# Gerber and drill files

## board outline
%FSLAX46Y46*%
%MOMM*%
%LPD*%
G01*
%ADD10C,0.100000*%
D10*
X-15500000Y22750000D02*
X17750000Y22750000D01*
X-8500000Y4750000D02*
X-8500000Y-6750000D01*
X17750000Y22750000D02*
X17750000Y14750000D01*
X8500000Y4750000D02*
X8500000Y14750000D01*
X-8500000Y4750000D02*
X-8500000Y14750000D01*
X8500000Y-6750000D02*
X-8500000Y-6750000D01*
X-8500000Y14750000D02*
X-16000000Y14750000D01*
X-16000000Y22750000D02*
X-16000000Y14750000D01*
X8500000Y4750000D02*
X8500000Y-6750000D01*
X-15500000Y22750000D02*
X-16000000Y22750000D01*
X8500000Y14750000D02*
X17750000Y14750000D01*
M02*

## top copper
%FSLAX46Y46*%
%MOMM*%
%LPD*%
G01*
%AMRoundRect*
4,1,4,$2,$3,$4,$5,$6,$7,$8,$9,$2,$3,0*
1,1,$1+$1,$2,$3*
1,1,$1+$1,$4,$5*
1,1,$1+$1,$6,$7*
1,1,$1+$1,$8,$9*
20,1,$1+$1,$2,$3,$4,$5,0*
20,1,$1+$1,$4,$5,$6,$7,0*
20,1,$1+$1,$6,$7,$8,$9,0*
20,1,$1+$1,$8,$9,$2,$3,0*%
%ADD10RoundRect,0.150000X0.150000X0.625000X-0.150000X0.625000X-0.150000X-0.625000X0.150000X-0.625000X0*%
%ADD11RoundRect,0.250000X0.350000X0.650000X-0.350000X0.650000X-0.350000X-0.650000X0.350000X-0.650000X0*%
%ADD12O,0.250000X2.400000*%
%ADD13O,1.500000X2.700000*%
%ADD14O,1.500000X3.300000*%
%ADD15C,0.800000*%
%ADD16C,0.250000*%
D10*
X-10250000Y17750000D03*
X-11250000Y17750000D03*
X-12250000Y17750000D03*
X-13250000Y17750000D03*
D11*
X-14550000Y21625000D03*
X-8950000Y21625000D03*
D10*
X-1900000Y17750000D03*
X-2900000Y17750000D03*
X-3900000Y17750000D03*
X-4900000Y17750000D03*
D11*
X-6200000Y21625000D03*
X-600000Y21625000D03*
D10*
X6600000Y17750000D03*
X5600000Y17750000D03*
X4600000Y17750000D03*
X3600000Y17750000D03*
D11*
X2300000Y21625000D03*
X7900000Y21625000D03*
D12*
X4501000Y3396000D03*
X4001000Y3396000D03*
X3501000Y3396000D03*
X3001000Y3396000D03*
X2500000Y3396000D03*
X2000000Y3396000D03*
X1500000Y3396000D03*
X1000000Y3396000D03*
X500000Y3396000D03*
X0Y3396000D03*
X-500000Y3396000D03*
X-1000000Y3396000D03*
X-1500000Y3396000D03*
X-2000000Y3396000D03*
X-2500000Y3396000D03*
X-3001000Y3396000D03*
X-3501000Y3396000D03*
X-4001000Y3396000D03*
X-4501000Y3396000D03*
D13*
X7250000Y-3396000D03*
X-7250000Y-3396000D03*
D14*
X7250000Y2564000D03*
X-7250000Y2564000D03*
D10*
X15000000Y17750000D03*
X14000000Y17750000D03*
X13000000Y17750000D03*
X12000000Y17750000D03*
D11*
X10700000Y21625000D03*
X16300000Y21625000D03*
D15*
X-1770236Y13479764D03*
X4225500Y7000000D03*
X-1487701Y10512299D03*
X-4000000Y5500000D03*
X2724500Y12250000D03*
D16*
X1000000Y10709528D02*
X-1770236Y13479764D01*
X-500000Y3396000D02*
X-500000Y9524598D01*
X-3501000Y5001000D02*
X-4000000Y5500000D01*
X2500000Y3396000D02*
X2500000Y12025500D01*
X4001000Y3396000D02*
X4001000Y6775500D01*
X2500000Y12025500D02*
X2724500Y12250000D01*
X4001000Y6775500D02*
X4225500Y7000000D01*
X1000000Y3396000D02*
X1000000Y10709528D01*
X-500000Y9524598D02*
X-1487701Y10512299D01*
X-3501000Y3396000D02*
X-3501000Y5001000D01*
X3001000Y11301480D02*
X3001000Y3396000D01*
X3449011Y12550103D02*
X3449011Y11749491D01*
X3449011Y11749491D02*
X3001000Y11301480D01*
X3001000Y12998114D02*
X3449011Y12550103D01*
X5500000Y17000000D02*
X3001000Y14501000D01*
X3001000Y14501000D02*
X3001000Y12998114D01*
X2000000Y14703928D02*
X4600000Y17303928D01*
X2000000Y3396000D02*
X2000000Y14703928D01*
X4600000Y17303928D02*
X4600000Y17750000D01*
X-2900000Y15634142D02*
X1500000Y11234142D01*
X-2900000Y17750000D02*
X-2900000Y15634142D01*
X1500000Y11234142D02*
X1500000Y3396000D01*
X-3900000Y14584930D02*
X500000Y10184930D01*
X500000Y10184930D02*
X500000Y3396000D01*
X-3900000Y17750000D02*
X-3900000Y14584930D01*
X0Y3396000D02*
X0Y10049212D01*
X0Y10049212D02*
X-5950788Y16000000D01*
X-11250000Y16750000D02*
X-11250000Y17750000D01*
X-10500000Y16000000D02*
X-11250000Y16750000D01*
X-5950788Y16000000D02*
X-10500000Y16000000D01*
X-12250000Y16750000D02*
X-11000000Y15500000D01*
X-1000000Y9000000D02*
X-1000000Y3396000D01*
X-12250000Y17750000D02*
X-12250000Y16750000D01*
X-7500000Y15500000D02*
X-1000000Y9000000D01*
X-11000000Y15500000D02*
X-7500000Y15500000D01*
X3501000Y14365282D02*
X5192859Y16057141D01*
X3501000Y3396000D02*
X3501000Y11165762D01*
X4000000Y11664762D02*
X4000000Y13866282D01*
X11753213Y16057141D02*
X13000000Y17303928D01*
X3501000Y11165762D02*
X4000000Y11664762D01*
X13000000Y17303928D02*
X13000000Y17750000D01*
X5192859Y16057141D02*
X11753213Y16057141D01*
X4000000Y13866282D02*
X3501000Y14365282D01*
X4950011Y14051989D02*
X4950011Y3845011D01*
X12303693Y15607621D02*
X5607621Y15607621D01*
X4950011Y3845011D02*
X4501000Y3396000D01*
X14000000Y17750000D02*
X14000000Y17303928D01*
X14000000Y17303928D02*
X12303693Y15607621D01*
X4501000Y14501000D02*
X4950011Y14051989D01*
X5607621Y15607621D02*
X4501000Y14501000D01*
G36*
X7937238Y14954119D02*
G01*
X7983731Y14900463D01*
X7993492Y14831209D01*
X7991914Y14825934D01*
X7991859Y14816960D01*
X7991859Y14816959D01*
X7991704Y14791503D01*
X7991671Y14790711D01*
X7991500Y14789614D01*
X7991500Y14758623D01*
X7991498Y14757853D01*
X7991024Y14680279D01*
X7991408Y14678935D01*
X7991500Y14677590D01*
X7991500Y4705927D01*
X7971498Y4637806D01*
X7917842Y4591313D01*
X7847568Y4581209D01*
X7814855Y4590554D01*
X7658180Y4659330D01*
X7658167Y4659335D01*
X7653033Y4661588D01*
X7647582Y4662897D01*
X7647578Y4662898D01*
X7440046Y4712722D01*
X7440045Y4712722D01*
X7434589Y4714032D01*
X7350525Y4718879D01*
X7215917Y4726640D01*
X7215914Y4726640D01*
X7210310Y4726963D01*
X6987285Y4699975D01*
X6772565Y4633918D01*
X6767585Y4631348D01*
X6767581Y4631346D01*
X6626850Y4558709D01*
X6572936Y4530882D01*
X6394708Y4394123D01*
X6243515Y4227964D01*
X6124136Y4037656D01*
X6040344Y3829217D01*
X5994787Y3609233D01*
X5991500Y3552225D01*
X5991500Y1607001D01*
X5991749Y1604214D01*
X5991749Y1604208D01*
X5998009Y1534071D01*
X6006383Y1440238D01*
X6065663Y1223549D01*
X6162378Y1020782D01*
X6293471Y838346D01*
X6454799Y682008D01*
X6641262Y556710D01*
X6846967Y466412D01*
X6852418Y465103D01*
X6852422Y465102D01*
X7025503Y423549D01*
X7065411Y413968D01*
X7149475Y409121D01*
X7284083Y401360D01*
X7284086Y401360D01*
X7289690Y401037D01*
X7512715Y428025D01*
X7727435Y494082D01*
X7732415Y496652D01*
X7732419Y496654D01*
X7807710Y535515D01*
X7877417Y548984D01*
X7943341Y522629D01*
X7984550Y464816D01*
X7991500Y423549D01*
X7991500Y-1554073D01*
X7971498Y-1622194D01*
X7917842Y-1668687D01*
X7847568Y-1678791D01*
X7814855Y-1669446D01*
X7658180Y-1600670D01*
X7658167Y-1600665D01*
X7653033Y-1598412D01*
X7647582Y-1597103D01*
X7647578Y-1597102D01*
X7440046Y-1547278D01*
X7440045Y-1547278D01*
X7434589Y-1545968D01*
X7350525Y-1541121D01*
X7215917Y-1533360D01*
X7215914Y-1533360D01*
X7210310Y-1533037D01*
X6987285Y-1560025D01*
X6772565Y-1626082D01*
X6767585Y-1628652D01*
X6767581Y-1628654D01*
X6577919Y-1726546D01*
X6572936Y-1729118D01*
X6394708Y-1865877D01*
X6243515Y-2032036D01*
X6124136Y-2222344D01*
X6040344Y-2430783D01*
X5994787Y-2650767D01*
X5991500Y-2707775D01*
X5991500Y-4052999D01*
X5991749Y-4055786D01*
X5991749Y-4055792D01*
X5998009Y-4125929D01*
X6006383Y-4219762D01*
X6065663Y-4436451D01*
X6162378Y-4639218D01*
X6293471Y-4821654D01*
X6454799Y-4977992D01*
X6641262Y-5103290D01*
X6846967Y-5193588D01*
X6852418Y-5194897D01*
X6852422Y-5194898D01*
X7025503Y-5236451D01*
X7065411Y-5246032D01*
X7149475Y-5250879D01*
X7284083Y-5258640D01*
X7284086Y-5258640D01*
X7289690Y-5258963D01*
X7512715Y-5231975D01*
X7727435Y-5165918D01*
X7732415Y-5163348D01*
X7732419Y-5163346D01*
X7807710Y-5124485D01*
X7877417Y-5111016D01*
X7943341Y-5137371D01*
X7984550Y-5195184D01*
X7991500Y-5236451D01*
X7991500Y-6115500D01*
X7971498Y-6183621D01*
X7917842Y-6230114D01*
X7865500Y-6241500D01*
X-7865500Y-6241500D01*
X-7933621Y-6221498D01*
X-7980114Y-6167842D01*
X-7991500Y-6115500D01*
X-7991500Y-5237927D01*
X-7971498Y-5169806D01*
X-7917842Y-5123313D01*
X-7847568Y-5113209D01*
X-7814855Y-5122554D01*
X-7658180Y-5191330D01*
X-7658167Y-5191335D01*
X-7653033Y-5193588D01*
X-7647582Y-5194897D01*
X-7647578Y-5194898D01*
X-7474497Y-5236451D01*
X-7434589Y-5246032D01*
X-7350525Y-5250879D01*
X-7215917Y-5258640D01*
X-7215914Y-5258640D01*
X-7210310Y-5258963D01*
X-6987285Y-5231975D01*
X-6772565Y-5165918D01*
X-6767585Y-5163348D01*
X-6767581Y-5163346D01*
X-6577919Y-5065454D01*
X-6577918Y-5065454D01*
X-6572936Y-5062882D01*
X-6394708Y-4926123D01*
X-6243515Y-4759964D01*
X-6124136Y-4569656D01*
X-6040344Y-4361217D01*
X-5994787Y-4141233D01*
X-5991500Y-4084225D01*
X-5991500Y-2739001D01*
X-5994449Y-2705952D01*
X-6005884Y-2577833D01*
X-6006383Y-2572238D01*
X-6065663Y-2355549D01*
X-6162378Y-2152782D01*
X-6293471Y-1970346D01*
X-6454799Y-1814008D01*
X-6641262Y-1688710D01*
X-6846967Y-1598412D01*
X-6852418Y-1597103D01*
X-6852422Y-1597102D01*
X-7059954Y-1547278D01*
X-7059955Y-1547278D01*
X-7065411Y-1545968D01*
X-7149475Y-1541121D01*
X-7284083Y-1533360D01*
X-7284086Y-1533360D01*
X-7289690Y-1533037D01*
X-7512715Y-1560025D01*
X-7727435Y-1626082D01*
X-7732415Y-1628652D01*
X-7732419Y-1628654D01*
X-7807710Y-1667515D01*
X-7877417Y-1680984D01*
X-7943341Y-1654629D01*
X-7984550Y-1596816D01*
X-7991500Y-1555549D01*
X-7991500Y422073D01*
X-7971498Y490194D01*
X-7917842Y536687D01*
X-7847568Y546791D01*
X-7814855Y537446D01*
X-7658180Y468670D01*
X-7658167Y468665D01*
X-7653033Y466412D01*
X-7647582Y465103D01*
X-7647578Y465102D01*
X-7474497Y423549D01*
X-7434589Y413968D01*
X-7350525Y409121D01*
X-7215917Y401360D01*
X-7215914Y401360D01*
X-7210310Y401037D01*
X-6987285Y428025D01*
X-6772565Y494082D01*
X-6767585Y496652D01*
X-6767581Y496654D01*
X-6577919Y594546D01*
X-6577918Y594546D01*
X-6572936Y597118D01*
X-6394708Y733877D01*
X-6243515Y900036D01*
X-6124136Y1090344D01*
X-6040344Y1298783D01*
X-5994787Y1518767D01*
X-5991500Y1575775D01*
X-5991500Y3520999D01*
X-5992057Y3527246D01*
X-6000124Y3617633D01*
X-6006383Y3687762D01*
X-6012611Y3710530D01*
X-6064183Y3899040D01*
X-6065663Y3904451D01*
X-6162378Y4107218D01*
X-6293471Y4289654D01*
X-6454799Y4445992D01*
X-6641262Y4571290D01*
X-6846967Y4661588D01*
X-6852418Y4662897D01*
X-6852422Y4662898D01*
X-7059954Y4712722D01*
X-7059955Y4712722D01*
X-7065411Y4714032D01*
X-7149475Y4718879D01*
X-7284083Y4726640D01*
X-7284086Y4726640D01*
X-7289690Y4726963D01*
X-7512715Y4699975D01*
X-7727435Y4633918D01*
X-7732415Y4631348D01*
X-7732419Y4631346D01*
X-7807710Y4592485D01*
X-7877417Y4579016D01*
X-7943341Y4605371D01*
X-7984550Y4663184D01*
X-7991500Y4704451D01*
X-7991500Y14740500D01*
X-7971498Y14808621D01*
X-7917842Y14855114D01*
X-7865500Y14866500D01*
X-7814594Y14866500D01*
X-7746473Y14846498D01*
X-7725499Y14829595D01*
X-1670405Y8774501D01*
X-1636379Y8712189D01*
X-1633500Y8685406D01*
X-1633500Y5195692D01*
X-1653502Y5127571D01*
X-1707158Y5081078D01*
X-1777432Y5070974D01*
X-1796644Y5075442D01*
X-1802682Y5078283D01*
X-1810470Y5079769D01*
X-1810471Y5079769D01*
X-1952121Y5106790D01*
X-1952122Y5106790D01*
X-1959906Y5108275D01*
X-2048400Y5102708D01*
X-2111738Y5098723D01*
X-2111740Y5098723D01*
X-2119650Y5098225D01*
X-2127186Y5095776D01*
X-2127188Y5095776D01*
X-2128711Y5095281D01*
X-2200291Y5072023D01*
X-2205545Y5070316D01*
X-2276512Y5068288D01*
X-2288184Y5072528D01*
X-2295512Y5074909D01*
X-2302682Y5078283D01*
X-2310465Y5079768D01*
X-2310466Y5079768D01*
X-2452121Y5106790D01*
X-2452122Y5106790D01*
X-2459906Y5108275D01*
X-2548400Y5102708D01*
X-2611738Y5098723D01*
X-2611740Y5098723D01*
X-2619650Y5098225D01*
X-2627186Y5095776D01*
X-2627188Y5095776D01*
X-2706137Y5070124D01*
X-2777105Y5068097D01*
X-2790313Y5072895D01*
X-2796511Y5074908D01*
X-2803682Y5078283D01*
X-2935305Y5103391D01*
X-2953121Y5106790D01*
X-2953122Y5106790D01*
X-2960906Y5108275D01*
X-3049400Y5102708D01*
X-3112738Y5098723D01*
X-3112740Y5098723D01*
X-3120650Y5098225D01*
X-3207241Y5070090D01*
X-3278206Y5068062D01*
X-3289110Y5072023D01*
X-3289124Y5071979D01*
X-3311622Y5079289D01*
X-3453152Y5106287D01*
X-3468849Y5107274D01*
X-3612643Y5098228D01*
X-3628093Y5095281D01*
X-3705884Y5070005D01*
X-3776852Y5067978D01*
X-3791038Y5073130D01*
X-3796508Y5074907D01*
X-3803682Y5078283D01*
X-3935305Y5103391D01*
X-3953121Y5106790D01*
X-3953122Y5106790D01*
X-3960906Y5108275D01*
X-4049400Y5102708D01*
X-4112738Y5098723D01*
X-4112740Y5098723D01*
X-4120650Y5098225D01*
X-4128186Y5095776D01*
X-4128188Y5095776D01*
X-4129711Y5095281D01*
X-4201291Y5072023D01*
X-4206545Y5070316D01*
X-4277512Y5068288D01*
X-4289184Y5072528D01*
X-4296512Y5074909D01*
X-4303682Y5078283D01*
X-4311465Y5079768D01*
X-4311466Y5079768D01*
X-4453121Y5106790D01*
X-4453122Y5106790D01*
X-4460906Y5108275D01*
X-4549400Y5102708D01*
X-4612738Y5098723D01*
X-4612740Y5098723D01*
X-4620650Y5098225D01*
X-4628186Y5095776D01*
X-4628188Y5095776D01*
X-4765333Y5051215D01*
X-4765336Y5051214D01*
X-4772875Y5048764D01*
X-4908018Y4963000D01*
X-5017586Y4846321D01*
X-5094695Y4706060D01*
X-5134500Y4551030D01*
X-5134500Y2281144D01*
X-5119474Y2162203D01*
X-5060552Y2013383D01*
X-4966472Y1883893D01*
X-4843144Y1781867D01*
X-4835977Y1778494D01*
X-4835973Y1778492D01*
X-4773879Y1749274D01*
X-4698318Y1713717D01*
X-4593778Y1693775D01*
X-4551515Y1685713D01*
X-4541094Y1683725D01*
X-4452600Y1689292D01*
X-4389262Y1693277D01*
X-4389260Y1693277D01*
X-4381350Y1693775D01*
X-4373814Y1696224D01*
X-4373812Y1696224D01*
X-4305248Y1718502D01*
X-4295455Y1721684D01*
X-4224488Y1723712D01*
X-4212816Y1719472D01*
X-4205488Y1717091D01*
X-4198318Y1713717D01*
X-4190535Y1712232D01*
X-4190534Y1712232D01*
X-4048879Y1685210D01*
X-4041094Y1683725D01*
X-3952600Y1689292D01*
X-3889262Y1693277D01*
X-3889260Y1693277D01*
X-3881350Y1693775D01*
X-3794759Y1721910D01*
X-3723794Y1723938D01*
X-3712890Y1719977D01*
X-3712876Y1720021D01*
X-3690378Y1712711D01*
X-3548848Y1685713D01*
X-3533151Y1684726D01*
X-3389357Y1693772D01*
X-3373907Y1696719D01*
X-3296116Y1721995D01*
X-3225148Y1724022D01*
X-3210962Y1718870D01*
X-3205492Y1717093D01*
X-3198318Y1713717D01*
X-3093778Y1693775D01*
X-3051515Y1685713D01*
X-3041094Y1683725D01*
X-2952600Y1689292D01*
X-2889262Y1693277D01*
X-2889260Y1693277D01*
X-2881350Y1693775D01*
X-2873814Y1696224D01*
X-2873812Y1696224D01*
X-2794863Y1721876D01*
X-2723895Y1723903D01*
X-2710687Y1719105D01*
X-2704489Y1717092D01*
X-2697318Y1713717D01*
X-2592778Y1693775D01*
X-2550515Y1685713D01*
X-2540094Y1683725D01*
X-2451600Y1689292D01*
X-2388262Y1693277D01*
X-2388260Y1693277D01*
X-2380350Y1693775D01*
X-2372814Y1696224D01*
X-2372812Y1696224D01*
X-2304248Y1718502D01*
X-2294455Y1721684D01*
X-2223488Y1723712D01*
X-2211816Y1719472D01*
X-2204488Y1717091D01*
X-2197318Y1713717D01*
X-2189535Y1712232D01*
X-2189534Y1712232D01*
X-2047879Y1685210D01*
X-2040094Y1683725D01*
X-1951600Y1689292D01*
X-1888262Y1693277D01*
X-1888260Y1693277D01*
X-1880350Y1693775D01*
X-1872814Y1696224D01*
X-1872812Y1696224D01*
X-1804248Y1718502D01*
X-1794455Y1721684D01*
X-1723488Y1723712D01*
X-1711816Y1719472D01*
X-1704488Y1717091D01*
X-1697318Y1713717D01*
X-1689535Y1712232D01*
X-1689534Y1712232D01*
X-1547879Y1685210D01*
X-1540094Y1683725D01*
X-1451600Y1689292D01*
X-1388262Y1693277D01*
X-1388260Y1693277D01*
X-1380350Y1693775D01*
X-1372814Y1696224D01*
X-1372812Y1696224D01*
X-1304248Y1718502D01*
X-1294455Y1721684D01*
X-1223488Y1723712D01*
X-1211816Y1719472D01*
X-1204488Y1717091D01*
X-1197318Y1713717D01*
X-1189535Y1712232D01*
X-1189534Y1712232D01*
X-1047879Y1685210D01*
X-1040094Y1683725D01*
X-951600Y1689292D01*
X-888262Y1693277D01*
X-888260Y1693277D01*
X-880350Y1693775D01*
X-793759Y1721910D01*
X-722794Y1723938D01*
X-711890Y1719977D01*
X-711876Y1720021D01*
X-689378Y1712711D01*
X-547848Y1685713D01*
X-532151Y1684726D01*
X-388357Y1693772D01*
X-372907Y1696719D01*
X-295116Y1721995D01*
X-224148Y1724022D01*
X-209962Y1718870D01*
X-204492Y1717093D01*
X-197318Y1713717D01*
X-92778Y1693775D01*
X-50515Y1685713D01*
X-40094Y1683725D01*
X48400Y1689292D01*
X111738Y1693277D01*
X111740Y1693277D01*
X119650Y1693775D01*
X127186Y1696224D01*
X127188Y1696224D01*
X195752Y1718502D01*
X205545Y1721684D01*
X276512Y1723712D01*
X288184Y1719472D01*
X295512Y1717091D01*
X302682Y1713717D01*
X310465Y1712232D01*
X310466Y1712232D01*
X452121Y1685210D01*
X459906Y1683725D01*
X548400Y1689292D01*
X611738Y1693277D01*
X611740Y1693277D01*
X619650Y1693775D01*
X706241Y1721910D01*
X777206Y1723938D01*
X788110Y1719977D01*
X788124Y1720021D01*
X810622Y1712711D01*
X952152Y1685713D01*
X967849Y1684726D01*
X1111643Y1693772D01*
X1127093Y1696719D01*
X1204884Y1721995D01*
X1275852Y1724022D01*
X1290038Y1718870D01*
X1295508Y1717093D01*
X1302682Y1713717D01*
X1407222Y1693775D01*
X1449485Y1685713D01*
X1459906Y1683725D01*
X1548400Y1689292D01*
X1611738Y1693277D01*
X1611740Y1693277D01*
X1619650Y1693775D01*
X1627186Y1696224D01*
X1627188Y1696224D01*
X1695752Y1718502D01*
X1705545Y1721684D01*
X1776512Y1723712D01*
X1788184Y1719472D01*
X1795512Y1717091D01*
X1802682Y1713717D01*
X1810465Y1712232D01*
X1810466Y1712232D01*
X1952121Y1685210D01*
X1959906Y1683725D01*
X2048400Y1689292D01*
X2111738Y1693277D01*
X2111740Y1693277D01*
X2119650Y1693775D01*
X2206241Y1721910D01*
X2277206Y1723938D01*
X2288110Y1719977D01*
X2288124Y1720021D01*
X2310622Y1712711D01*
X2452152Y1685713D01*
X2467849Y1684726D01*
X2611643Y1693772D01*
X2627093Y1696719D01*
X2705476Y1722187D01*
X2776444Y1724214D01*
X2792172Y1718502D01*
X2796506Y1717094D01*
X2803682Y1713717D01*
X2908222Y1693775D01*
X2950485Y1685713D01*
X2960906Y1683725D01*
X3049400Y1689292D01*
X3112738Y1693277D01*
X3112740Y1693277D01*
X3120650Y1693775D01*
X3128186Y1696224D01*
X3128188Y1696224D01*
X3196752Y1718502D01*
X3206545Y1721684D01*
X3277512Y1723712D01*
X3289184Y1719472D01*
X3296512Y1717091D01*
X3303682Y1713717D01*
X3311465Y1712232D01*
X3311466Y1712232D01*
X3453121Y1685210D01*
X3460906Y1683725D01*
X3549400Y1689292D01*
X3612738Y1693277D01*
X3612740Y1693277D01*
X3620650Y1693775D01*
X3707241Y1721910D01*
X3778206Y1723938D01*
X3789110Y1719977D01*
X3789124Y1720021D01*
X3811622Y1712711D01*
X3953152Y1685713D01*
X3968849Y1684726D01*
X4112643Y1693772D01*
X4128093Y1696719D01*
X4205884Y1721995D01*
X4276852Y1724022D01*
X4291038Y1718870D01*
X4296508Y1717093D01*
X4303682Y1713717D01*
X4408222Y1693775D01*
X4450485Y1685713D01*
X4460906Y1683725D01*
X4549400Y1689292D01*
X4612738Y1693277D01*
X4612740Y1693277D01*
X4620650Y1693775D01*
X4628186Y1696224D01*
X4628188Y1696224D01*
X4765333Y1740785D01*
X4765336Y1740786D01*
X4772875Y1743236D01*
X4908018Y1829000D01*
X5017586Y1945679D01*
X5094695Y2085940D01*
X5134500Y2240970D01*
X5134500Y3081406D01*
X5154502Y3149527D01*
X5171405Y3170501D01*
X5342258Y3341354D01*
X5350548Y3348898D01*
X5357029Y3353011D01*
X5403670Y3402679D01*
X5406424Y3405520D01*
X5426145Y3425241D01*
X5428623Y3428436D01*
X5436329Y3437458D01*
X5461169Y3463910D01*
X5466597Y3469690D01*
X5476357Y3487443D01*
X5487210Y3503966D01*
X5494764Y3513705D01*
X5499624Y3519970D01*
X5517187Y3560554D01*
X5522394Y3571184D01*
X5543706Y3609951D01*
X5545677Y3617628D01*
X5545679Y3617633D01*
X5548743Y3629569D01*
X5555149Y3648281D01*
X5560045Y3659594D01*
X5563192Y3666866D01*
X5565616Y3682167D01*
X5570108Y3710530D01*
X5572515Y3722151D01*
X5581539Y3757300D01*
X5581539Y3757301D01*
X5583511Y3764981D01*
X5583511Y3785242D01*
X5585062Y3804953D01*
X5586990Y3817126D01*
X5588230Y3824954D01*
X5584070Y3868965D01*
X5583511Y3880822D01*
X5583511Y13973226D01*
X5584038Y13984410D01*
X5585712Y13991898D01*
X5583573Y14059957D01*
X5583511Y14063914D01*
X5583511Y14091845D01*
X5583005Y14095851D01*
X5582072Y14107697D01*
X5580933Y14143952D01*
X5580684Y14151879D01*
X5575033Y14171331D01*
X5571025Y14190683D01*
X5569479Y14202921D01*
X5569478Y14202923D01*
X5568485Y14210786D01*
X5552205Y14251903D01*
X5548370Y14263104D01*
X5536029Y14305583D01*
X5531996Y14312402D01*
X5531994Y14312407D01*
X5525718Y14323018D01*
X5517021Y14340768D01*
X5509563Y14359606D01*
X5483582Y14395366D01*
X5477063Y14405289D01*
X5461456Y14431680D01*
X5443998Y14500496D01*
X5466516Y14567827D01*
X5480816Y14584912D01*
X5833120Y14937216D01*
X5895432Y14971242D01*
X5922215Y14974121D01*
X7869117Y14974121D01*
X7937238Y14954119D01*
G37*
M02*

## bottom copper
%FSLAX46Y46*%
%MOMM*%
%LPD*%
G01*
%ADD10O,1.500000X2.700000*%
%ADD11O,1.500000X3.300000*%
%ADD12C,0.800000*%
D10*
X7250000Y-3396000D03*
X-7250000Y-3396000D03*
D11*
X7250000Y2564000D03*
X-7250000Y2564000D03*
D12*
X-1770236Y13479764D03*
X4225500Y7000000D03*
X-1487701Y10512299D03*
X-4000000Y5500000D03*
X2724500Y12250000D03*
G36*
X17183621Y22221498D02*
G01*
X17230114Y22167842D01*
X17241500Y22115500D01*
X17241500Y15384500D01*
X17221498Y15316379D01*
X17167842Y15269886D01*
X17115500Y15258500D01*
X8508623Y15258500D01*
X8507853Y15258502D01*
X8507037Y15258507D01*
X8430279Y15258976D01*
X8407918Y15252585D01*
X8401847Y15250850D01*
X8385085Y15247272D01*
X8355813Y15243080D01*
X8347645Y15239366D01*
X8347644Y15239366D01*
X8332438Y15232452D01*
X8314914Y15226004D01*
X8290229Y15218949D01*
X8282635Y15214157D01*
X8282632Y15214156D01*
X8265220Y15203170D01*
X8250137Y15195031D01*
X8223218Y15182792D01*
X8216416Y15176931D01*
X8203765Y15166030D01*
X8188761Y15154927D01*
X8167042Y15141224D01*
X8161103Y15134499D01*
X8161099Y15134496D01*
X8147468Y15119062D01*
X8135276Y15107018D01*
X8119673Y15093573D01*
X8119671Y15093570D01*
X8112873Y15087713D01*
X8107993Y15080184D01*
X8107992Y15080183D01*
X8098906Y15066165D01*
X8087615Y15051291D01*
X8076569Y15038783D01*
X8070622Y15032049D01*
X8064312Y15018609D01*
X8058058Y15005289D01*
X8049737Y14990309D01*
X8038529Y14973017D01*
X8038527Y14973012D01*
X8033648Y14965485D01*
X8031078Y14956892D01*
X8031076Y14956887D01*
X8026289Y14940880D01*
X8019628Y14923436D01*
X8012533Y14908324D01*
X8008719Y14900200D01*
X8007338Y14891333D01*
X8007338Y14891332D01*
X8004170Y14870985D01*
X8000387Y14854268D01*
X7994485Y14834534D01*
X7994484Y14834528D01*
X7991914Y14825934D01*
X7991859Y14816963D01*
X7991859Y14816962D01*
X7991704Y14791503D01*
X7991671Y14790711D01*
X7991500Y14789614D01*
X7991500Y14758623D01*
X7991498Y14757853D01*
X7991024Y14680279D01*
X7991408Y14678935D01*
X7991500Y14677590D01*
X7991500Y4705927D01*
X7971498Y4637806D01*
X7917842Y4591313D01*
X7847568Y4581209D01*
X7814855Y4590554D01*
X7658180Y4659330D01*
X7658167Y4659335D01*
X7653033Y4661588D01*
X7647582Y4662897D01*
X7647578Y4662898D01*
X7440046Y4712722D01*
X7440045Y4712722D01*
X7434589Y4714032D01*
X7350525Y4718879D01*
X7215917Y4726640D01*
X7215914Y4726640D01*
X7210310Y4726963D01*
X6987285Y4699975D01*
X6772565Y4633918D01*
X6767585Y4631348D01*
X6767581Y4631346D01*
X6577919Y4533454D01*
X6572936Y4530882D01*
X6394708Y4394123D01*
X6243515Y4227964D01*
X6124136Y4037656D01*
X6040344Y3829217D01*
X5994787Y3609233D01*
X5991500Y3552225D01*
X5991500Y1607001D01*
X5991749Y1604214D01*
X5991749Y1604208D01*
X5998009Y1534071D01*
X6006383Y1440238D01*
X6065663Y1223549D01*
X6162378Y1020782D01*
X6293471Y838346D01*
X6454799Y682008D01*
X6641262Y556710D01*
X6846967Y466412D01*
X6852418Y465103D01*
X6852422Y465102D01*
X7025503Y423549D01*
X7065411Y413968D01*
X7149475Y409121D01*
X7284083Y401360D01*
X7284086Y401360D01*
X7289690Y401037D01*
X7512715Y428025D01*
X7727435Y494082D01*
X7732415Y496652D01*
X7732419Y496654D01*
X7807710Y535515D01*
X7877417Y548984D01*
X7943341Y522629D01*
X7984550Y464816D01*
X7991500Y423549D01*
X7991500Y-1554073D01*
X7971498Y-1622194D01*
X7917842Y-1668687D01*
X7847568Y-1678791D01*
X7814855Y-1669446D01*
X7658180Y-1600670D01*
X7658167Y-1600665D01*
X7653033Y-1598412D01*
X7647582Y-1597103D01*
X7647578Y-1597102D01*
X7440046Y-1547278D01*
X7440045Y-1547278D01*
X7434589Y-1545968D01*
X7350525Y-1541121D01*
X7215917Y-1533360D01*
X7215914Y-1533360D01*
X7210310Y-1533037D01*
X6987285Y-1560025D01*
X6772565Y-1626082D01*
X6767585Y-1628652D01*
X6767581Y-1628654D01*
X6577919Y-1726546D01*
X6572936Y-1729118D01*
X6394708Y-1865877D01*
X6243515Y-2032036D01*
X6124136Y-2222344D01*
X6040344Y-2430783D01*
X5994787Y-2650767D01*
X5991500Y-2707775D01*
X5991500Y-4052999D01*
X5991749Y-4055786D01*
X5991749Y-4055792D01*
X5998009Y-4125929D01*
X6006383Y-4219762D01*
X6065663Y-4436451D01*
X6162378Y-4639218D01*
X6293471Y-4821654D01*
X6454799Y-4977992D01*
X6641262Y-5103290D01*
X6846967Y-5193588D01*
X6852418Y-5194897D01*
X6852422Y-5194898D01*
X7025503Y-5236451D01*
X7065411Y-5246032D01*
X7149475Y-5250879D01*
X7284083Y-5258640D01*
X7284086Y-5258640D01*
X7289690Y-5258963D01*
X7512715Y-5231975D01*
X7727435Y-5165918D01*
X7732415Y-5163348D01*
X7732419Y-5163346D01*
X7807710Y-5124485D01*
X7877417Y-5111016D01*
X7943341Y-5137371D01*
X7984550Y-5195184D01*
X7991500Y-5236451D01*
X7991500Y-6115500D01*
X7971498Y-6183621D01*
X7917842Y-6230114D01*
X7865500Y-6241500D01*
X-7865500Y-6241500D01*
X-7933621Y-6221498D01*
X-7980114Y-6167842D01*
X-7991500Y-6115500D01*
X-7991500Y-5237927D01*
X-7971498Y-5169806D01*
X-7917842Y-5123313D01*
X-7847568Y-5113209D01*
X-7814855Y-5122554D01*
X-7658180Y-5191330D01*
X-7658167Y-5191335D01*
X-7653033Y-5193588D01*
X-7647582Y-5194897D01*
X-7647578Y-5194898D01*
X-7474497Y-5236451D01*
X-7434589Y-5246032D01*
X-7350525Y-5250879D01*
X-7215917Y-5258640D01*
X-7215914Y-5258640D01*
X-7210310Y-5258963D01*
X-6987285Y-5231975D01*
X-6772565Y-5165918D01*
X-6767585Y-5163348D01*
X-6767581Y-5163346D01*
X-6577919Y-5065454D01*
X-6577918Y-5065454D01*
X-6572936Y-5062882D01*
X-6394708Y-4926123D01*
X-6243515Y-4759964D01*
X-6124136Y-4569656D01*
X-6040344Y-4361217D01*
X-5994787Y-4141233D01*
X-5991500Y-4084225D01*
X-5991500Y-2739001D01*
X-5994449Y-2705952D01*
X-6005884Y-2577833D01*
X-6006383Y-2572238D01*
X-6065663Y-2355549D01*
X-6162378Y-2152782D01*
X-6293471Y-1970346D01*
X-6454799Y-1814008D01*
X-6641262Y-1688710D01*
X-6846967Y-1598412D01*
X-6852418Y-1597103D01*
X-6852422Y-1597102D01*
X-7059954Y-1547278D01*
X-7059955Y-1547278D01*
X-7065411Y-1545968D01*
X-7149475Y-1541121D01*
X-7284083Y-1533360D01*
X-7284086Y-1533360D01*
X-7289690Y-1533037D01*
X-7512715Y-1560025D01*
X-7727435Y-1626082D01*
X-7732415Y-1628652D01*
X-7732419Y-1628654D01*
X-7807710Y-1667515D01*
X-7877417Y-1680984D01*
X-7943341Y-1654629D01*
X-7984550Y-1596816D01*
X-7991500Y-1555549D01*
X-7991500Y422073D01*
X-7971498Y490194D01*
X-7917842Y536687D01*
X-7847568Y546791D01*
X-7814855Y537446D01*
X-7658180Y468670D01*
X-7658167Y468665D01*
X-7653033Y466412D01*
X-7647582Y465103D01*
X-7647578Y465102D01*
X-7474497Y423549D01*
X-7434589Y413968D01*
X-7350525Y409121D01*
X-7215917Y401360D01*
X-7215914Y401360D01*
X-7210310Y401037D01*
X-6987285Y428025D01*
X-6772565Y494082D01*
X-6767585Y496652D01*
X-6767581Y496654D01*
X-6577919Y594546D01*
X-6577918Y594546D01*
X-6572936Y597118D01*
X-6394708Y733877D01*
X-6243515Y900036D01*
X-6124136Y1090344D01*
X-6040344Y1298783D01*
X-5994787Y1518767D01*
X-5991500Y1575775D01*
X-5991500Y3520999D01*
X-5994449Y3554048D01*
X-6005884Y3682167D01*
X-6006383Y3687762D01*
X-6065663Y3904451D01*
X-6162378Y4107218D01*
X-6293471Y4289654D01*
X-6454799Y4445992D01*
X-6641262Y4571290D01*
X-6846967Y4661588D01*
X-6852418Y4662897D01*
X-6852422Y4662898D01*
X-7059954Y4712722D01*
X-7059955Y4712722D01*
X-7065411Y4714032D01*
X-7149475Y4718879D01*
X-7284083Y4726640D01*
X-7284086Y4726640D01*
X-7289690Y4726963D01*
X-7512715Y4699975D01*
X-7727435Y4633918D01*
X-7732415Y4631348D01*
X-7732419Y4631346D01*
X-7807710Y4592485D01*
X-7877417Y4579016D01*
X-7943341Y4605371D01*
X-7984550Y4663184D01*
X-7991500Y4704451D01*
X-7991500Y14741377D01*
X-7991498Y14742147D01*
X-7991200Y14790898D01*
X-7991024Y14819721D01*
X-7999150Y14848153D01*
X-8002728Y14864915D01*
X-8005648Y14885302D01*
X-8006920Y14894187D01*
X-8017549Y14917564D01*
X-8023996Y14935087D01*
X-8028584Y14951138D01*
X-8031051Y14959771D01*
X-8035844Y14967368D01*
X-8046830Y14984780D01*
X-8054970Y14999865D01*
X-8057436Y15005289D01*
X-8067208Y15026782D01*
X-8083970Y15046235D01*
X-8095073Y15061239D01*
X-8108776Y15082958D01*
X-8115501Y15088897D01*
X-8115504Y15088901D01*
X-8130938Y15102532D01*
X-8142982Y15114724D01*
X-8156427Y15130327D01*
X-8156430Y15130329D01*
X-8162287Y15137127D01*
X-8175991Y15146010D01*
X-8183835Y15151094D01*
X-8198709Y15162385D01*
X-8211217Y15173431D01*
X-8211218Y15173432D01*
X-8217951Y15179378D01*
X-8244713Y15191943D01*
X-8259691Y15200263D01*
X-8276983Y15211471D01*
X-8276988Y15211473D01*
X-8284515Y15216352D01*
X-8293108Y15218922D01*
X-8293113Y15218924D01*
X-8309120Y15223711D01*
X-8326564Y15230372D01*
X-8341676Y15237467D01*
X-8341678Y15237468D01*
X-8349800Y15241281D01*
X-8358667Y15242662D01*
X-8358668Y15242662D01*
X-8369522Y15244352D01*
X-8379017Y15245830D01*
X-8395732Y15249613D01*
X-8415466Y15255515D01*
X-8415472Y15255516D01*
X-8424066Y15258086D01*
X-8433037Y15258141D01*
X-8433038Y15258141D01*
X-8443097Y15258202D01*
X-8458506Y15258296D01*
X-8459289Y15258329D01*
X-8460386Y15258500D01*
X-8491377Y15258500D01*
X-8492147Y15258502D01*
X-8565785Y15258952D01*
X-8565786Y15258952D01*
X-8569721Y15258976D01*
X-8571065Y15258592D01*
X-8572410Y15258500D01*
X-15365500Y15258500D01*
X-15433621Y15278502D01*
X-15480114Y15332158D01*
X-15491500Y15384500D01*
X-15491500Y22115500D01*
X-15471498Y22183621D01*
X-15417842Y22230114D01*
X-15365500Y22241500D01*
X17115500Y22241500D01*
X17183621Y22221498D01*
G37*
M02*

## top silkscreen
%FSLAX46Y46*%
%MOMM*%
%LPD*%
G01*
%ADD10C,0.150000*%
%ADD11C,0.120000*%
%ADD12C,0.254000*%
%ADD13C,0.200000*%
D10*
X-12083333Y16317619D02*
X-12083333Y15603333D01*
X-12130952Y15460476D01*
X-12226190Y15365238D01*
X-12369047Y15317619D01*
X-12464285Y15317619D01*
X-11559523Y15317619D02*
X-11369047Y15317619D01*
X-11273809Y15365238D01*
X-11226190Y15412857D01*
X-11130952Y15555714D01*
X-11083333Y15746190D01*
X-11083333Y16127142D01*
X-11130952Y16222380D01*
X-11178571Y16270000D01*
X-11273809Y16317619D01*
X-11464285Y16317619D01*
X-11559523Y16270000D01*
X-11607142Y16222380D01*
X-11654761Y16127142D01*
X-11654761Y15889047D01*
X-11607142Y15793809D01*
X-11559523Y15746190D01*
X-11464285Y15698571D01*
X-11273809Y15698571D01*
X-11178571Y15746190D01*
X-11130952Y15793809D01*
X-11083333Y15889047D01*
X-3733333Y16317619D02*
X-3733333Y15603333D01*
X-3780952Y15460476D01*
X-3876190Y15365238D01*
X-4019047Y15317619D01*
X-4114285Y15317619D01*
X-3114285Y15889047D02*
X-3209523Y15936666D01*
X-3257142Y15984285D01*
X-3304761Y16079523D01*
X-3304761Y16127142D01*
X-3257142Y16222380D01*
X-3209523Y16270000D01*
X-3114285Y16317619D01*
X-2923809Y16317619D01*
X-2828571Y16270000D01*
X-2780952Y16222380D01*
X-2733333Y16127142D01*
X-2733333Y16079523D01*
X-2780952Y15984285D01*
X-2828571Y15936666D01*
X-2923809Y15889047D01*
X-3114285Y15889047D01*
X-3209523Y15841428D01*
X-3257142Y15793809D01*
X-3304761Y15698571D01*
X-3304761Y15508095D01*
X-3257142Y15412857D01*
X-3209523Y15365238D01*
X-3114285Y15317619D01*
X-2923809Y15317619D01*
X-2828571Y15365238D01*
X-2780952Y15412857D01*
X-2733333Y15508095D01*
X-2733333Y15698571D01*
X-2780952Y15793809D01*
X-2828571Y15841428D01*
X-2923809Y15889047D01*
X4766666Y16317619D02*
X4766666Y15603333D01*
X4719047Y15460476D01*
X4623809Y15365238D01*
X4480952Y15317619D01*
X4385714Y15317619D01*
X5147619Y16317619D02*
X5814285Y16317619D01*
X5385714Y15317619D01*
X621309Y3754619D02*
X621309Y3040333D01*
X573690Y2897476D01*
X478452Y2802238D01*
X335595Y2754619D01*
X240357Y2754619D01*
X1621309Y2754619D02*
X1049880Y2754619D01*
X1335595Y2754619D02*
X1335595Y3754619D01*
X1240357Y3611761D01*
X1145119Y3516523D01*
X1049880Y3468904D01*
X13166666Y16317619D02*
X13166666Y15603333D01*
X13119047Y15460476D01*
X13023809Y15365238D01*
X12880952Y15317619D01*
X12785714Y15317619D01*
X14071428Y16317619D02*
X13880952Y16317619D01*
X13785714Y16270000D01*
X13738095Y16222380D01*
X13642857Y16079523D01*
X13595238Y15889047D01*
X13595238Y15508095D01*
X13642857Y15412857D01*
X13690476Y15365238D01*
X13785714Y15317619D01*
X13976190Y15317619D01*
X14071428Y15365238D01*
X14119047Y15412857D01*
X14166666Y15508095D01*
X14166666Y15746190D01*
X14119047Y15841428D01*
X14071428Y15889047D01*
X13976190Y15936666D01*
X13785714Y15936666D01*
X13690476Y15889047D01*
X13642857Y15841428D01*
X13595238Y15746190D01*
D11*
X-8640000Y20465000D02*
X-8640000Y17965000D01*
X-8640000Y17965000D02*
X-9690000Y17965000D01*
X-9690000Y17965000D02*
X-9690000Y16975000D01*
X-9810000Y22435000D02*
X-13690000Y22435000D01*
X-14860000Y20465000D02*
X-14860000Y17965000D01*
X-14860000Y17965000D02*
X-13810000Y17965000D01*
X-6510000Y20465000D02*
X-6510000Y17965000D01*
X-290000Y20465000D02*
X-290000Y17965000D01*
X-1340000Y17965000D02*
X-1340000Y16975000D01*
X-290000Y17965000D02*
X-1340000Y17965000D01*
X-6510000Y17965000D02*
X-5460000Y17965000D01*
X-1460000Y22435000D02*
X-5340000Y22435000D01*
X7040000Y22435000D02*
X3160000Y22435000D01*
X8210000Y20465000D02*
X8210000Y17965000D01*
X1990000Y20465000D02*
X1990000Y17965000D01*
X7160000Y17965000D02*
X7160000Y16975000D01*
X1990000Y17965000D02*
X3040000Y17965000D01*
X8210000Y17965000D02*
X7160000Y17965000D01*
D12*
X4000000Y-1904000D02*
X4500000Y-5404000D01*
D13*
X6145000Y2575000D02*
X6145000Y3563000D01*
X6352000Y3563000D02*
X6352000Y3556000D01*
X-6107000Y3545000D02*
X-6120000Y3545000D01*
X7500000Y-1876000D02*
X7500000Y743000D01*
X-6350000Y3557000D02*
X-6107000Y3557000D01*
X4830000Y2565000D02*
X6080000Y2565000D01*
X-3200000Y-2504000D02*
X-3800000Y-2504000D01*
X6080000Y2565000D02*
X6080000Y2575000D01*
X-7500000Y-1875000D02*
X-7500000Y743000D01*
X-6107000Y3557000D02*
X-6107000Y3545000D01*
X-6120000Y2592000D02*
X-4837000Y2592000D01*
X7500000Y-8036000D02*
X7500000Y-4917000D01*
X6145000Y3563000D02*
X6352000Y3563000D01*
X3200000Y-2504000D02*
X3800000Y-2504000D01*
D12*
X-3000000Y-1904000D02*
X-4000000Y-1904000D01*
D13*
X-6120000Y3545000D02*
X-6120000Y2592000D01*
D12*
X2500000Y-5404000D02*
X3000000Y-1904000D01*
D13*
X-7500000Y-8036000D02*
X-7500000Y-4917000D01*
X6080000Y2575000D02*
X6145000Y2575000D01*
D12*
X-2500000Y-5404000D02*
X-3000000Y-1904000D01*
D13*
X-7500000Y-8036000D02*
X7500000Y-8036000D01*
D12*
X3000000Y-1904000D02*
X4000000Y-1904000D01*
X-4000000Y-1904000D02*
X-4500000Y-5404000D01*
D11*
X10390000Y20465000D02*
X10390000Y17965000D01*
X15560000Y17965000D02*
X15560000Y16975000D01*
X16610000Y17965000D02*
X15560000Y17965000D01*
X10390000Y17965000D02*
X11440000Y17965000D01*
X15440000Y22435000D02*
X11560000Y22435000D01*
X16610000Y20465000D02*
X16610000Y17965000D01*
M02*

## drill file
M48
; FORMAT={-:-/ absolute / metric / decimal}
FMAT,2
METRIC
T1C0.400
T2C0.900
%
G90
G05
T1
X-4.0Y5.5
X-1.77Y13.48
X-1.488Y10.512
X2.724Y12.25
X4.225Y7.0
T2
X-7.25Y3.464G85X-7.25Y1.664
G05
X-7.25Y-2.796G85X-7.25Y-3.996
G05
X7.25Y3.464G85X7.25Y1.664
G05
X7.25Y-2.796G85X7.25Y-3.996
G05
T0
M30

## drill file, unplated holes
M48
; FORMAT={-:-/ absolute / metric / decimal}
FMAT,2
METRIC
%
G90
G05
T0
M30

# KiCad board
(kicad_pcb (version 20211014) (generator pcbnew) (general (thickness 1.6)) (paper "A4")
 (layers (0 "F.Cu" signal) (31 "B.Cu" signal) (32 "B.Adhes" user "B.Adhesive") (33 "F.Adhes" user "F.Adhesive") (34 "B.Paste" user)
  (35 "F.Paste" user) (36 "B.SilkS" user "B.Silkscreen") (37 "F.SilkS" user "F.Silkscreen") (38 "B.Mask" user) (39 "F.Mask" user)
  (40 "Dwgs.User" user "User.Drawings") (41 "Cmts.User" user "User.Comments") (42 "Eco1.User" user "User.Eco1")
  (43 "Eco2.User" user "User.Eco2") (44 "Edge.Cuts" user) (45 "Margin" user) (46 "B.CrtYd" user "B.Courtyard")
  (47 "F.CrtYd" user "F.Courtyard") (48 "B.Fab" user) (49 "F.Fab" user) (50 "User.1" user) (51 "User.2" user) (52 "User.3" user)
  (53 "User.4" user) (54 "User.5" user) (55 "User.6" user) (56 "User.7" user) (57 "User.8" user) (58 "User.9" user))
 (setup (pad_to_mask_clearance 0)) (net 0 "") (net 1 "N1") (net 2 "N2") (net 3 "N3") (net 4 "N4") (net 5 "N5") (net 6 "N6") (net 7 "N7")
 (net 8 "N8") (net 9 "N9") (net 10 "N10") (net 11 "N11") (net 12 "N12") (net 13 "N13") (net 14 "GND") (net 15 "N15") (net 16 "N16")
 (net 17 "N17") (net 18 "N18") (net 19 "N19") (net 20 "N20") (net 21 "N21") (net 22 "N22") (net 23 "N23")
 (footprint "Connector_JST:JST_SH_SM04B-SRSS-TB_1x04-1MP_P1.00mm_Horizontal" (layer "F.Cu") (at -11.75 -19.75 180)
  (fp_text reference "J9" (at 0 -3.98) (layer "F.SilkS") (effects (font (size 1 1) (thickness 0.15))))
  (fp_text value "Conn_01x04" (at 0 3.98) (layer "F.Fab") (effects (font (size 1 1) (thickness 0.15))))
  (fp_line (start -3.11 0.715) (end -3.11 -1.785) (layer "F.SilkS") (width 0.12))
  (fp_line (start -3.11 -1.785) (end -2.06 -1.785) (layer "F.SilkS") (width 0.12))
  (fp_line (start -2.06 -1.785) (end -2.06 -2.775) (layer "F.SilkS") (width 0.12))
  (fp_line (start -1.94 2.685) (end 1.94 2.685) (layer "F.SilkS") (width 0.12))
  (fp_line (start 3.11 0.715) (end 3.11 -1.785) (layer "F.SilkS") (width 0.12))
  (fp_line (start 3.11 -1.785) (end 2.06 -1.785) (layer "F.SilkS") (width 0.12))
  (pad "1" smd roundrect (at -1.5 -2 180) (size 0.6 1.55) (layers "F.Cu" "F.Paste" "F.Mask") (roundrect_rratio 0.25) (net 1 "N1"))
  (pad "2" smd roundrect (at -0.5 -2 180) (size 0.6 1.55) (layers "F.Cu" "F.Paste" "F.Mask") (roundrect_rratio 0.25) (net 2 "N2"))
  (pad "3" smd roundrect (at 0.5 -2 180) (size 0.6 1.55) (layers "F.Cu" "F.Paste" "F.Mask") (roundrect_rratio 0.25) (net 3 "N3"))
  (pad "4" smd roundrect (at 1.5 -2 180) (size 0.6 1.55) (layers "F.Cu" "F.Paste" "F.Mask") (roundrect_rratio 0.25) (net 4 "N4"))
  (pad "MP" smd roundrect (at 2.8 1.875 180) (size 1.2 1.8) (layers "F.Cu" "F.Paste" "F.Mask") (roundrect_rratio 0.2083333333))
  (pad "MP" smd roundrect (at -2.8 1.875 180) (size 1.2 1.8) (layers "F.Cu" "F.Paste" "F.Mask") (roundrect_rratio 0.2083333333)))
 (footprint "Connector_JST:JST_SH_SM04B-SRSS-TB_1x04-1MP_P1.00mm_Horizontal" (layer "F.Cu") (at -3.4 -19.75 180)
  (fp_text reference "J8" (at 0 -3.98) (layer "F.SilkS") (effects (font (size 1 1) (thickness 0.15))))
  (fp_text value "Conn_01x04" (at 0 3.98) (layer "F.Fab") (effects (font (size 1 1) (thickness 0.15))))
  (fp_line (start 3.11 0.715) (end 3.11 -1.785) (layer "F.SilkS") (width 0.12))
  (fp_line (start -3.11 0.715) (end -3.11 -1.785) (layer "F.SilkS") (width 0.12))
  (fp_line (start -2.06 -1.785) (end -2.06 -2.775) (layer "F.SilkS") (width 0.12))
  (fp_line (start -3.11 -1.785) (end -2.06 -1.785) (layer "F.SilkS") (width 0.12))
  (fp_line (start 3.11 -1.785) (end 2.06 -1.785) (layer "F.SilkS") (width 0.12))
  (fp_line (start -1.94 2.685) (end 1.94 2.685) (layer "F.SilkS") (width 0.12))
  (pad "1" smd roundrect (at -1.5 -2 180) (size 0.6 1.55) (layers "F.Cu" "F.Paste" "F.Mask") (roundrect_rratio 0.25) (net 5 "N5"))
  (pad "2" smd roundrect (at -0.5 -2 180) (size 0.6 1.55) (layers "F.Cu" "F.Paste" "F.Mask") (roundrect_rratio 0.25) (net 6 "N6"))
  (pad "3" smd roundrect (at 0.5 -2 180) (size 0.6 1.55) (layers "F.Cu" "F.Paste" "F.Mask") (roundrect_rratio 0.25) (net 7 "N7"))
  (pad "4" smd roundrect (at 1.5 -2 180) (size 0.6 1.55) (layers "F.Cu" "F.Paste" "F.Mask") (roundrect_rratio 0.25) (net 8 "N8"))
  (pad "MP" smd roundrect (at 2.8 1.875 180) (size 1.2 1.8) (layers "F.Cu" "F.Paste" "F.Mask") (roundrect_rratio 0.2083333333))
  (pad "MP" smd roundrect (at -2.8 1.875 180) (size 1.2 1.8) (layers "F.Cu" "F.Paste" "F.Mask") (roundrect_rratio 0.2083333333)))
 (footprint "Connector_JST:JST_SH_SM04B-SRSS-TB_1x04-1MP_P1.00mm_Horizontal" (layer "F.Cu") (at 5.1 -19.75 180)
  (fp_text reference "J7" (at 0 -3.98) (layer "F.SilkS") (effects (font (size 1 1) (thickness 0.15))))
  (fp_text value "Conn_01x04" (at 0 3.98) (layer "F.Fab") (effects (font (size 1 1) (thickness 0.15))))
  (fp_line (start -1.94 2.685) (end 1.94 2.685) (layer "F.SilkS") (width 0.12))
  (fp_line (start -3.11 0.715) (end -3.11 -1.785) (layer "F.SilkS") (width 0.12))
  (fp_line (start 3.11 0.715) (end 3.11 -1.785) (layer "F.SilkS") (width 0.12))
  (fp_line (start -2.06 -1.785) (end -2.06 -2.775) (layer "F.SilkS") (width 0.12))
  (fp_line (start 3.11 -1.785) (end 2.06 -1.785) (layer "F.SilkS") (width 0.12))
  (fp_line (start -3.11 -1.785) (end -2.06 -1.785) (layer "F.SilkS") (width 0.12))
  (pad "1" smd roundrect (at -1.5 -2 180) (size 0.6 1.55) (layers "F.Cu" "F.Paste" "F.Mask") (roundrect_rratio 0.25) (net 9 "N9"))
  (pad "2" smd roundrect (at -0.5 -2 180) (size 0.6 1.55) (layers "F.Cu" "F.Paste" "F.Mask") (roundrect_rratio 0.25) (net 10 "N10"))
  (pad "3" smd roundrect (at 0.5 -2 180) (size 0.6 1.55) (layers "F.Cu" "F.Paste" "F.Mask") (roundrect_rratio 0.25) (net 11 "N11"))
  (pad "4" smd roundrect (at 1.5 -2 180) (size 0.6 1.55) (layers "F.Cu" "F.Paste" "F.Mask") (roundrect_rratio 0.25) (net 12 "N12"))
  (pad "MP" smd roundrect (at 2.8 1.875 180) (size 1.2 1.8) (layers "F.Cu" "F.Paste" "F.Mask") (roundrect_rratio 0.2083333333))
  (pad "MP" smd roundrect (at -2.8 1.875 180) (size 1.2 1.8) (layers "F.Cu" "F.Paste" "F.Mask") (roundrect_rratio 0.2083333333)))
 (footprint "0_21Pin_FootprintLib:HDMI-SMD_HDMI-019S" (layer "F.Cu") (at 0 0)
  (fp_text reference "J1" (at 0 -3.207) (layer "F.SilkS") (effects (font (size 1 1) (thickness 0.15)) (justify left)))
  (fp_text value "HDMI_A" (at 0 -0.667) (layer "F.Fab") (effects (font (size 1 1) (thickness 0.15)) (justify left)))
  (fp_line (start 4 1.904) (end 4.5 5.404) (layer "F.SilkS") (width 0.254))
  (fp_line (start 6.145 -2.575) (end 6.145 -3.563) (layer "F.SilkS") (width 0.2))
  (fp_line (start 6.352 -3.563) (end 6.352 -3.556) (layer "F.SilkS") (width 0.2))
  (fp_line (start -6.107 -3.545) (end -6.12 -3.545) (layer "F.SilkS") (width 0.2))
  (fp_line (start 7.5 1.876) (end 7.5 -0.743) (layer "F.SilkS") (width 0.2))
  (fp_line (start -6.35 -3.557) (end -6.107 -3.557) (layer "F.SilkS") (width 0.2))
  (fp_line (start 4.83 -2.565) (end 6.08 -2.565) (layer "F.SilkS") (width 0.2))
  (fp_line (start -3.2 2.504) (end -3.8 2.504) (layer "F.SilkS") (width 0.2))
  (fp_line (start 6.08 -2.565) (end 6.08 -2.575) (layer "F.SilkS") (width 0.2))
  (fp_line (start -7.5 1.875) (end -7.5 -0.743) (layer "F.SilkS") (width 0.2))
  (fp_line (start -6.107 -3.557) (end -6.107 -3.545) (layer "F.SilkS") (width 0.2))
  (fp_line (start -6.12 -2.592) (end -4.837 -2.592) (layer "F.SilkS") (width 0.2))
  (fp_line (start 7.5 8.036) (end 7.5 4.917) (layer "F.SilkS") (width 0.2))
  (fp_line (start 6.145 -3.563) (end 6.352 -3.563) (layer "F.SilkS") (width 0.2))
  (fp_line (start 3.2 2.504) (end 3.8 2.504) (layer "F.SilkS") (width 0.2))
  (fp_line (start -3 1.904) (end -4 1.904) (layer "F.SilkS") (width 0.254))
  (fp_line (start -6.12 -3.545) (end -6.12 -2.592) (layer "F.SilkS") (width 0.2))
  (fp_line (start 2.5 5.404) (end 3 1.904) (layer "F.SilkS") (width 0.254))
  (fp_line (start -7.5 8.036) (end -7.5 4.917) (layer "F.SilkS") (width 0.2))
  (fp_line (start 6.08 -2.575) (end 6.145 -2.575) (layer "F.SilkS") (width 0.2))
  (fp_line (start -2.5 5.404) (end -3 1.904) (layer "F.SilkS") (width 0.254))
  (fp_line (start -7.5 8.036) (end 7.5 8.036) (layer "F.SilkS") (width 0.2))
  (fp_line (start 3 1.904) (end 4 1.904) (layer "F.SilkS") (width 0.254))
  (fp_line (start -4 1.904) (end -4.5 5.404) (layer "F.SilkS") (width 0.254))
  (pad "1" smd oval (at 4.501 -3.396) (size 0.25 2.4) (layers "F.Cu" "F.Paste" "F.Mask") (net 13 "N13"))
  (pad "2" smd oval (at 4.001 -3.396) (size 0.25 2.4) (layers "F.Cu" "F.Paste" "F.Mask") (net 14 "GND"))
  (pad "3" smd oval (at 3.501 -3.396) (size 0.25 2.4) (layers "F.Cu" "F.Paste" "F.Mask") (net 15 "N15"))
  (pad "4" smd oval (at 3.001 -3.396) (size 0.25 2.4) (layers "F.Cu" "F.Paste" "F.Mask") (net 10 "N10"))
  (pad "5" smd oval (at 2.5 -3.396) (size 0.25 2.4) (layers "F.Cu" "F.Paste" "F.Mask") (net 14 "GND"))
  (pad "6" smd oval (at 2 -3.396) (size 0.25 2.4) (layers "F.Cu" "F.Paste" "F.Mask") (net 11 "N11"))
  (pad "7" smd oval (at 1.5 -3.396) (size 0.25 2.4) (layers "F.Cu" "F.Paste" "F.Mask") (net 6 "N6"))
  (pad "8" smd oval (at 1 -3.396) (size 0.25 2.4) (layers "F.Cu" "F.Paste" "F.Mask") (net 14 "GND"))
  (pad "9" smd oval (at 0.5 -3.396) (size 0.25 2.4) (layers "F.Cu" "F.Paste" "F.Mask") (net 7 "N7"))
  (pad "10" smd oval (at 0 -3.396) (size 0.25 2.4) (layers "F.Cu" "F.Paste" "F.Mask") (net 2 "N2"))
  (pad "11" smd oval (at -0.5 -3.396) (size 0.25 2.4) (layers "F.Cu" "F.Paste" "F.Mask") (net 14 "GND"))
  (pad "12" smd oval (at -1 -3.396) (size 0.25 2.4) (layers "F.Cu" "F.Paste" "F.Mask") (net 3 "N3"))
  (pad "13" smd oval (at -1.5 -3.396) (size 0.25 2.4) (layers "F.Cu" "F.Paste" "F.Mask") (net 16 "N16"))
  (pad "14" smd oval (at -2 -3.396) (size 0.25 2.4) (layers "F.Cu" "F.Paste" "F.Mask") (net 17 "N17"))
  (pad "15" smd oval (at -2.5 -3.396) (size 0.25 2.4) (layers "F.Cu" "F.Paste" "F.Mask") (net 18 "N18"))
  (pad "16" smd oval (at -3.001 -3.396) (size 0.25 2.4) (layers "F.Cu" "F.Paste" "F.Mask") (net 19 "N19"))
  (pad "17" smd oval (at -3.501 -3.396) (size 0.25 2.4) (layers "F.Cu" "F.Paste" "F.Mask") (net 14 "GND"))
  (pad "18" smd oval (at -4.001 -3.396) (size 0.25 2.4) (layers "F.Cu" "F.Paste" "F.Mask") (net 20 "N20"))
  (pad "19" smd oval (at -4.501 -3.396) (size 0.25 2.4) (layers "F.Cu" "F.Paste" "F.Mask") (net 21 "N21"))
  (pad "20" thru_hole oval (at 7.25 3.396) (size 1.5 2.7) (drill oval 0.9 2.1) (layers *.Cu *.Mask))
  (pad "21" thru_hole oval (at -7.25 3.396) (size 1.5 2.7) (drill oval 0.9 2.1) (layers *.Cu *.Mask))
  (pad "22" thru_hole oval (at 7.25 -2.564) (size 1.5 3.3) (drill oval 0.9 2.7) (layers *.Cu *.Mask))
  (pad "23" thru_hole oval (at -7.25 -2.564) (size 1.5 3.3) (drill oval 0.9 2.7) (layers *.Cu *.Mask)))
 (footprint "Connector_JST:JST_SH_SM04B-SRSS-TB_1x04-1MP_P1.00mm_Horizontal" (layer "F.Cu") (at 13.5 -19.75 180)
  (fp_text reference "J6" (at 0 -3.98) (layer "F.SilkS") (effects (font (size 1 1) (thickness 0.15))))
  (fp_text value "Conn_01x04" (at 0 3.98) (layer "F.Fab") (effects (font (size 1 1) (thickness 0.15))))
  (fp_line (start 3.11 0.715) (end 3.11 -1.785) (layer "F.SilkS") (width 0.12))
  (fp_line (start -2.06 -1.785) (end -2.06 -2.775) (layer "F.SilkS") (width 0.12))
  (fp_line (start -3.11 -1.785) (end -2.06 -1.785) (layer "F.SilkS") (width 0.12))
  (fp_line (start 3.11 -1.785) (end 2.06 -1.785) (layer "F.SilkS") (width 0.12))
  (fp_line (start -1.94 2.685) (end 1.94 2.685) (layer "F.SilkS") (width 0.12))
  (fp_line (start -3.11 0.715) (end -3.11 -1.785) (layer "F.SilkS") (width 0.12))
  (pad "1" smd roundrect (at -1.5 -2 180) (size 0.6 1.55) (layers "F.Cu" "F.Paste" "F.Mask") (roundrect_rratio 0.25) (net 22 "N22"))
  (pad "2" smd roundrect (at -0.5 -2 180) (size 0.6 1.55) (layers "F.Cu" "F.Paste" "F.Mask") (roundrect_rratio 0.25) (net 13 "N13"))
  (pad "3" smd roundrect (at 0.5 -2 180) (size 0.6 1.55) (layers "F.Cu" "F.Paste" "F.Mask") (roundrect_rratio 0.25) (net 15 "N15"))
  (pad "4" smd roundrect (at 1.5 -2 180) (size 0.6 1.55) (layers "F.Cu" "F.Paste" "F.Mask") (roundrect_rratio 0.25) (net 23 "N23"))
  (pad "MP" smd roundrect (at 2.8 1.875 180) (size 1.2 1.8) (layers "F.Cu" "F.Paste" "F.Mask") (roundrect_rratio 0.2083333333))
  (pad "MP" smd roundrect (at -2.8 1.875 180) (size 1.2 1.8) (layers "F.Cu" "F.Paste" "F.Mask") (roundrect_rratio 0.2083333333)))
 (gr_line (start -15.5 -22.75) (end 17.75 -22.75) (layer "Edge.Cuts") (width 0.1))
 (gr_line (start -8.5 -4.75) (end -8.5 6.75) (layer "Edge.Cuts") (width 0.1))
 (gr_line (start 17.75 -22.75) (end 17.75 -14.75) (layer "Edge.Cuts") (width 0.1))
 (gr_line (start 8.5 -4.75) (end 8.5 -14.75) (layer "Edge.Cuts") (width 0.1))
 (gr_line (start -8.5 -4.75) (end -8.5 -14.75) (layer "Edge.Cuts") (width 0.1))
 (gr_line (start 8.5 6.75) (end -8.5 6.75) (layer "Edge.Cuts") (width 0.1))
 (gr_line (start -8.5 -14.75) (end -16 -14.75) (layer "Edge.Cuts") (width 0.1))
 (gr_line (start -16 -22.75) (end -16 -14.75) (layer "Edge.Cuts") (width 0.1))
 (gr_line (start 8.5 -4.75) (end 8.5 6.75) (layer "Edge.Cuts") (width 0.1))
 (gr_line (start -15.5 -22.75) (end -16 -22.75) (layer "Edge.Cuts") (width 0.1))
 (gr_line (start 8.5 -14.75) (end 17.75 -14.75) (layer "Edge.Cuts") (width 0.1))
 (segment (start 1 -10.709528) (end -1.770236 -13.479764) (width 0.25) (layer "F.Cu") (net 14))
 (segment (start -0.5 -3.396) (end -0.5 -9.524598) (width 0.25) (layer "F.Cu") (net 14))
 (segment (start -3.501 -5.001) (end -4 -5.5) (width 0.25) (layer "F.Cu") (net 14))
 (segment (start 2.5 -3.396) (end 2.5 -12.0255) (width 0.25) (layer "F.Cu") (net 14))
 (segment (start 4.001 -3.396) (end 4.001 -6.7755) (width 0.25) (layer "F.Cu") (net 14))
 (segment (start 2.5 -12.0255) (end 2.7245 -12.25) (width 0.25) (layer "F.Cu") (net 14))
 (segment (start 4.001 -6.7755) (end 4.2255 -7) (width 0.25) (layer "F.Cu") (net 14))
 (segment (start 1 -3.396) (end 1 -10.709528) (width 0.25) (layer "F.Cu") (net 14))
 (segment (start -0.5 -9.524598) (end -1.487701 -10.512299) (width 0.25) (layer "F.Cu") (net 14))
 (segment (start -3.501 -3.396) (end -3.501 -5.001) (width 0.25) (layer "F.Cu") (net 14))
 (via (at -1.770236 -13.479764) (size 0.8) (drill 0.4) (layers "F.Cu" "B.Cu") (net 14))
 (via (at 4.2255 -7) (size 0.8) (drill 0.4) (layers "F.Cu" "B.Cu") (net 14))
 (via (at -1.487701 -10.512299) (size 0.8) (drill 0.4) (layers "F.Cu" "B.Cu") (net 14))
 (via (at -4 -5.5) (size 0.8) (drill 0.4) (layers "F.Cu" "B.Cu") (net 14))
 (via (at 2.7245 -12.25) (size 0.8) (drill 0.4) (layers "F.Cu" "B.Cu") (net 14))
 (segment (start 3.001 -11.30148) (end 3.001 -3.396) (width 0.25) (layer "F.Cu") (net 10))
 (segment (start 3.449011 -12.550103) (end 3.449011 -11.749491) (width 0.25) (layer "F.Cu") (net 10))
 (segment (start 3.449011 -11.749491) (end 3.001 -11.30148) (width 0.25) (layer "F.Cu") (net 10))
 (segment (start 3.001 -12.998114) (end 3.449011 -12.550103) (width 0.25) (layer "F.Cu") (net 10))
 (segment (start 5.5 -17) (end 3.001 -14.501) (width 0.25) (layer "F.Cu") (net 10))
 (segment (start 3.001 -14.501) (end 3.001 -12.998114) (width 0.25) (layer "F.Cu") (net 10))
 (segment (start 2 -14.703928) (end 4.6 -17.303928) (width 0.25) (layer "F.Cu") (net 11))
 (segment (start 2 -3.396) (end 2 -14.703928) (width 0.25) (layer "F.Cu") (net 11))
 (segment (start 4.6 -17.303928) (end 4.6 -17.75) (width 0.25) (layer "F.Cu") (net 11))
 (segment (start -2.9 -15.634142) (end 1.5 -11.234142) (width 0.25) (layer "F.Cu") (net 6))
 (segment (start -2.9 -17.75) (end -2.9 -15.634142) (width 0.25) (layer "F.Cu") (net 6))
 (segment (start 1.5 -11.234142) (end 1.5 -3.396) (width 0.25) (layer "F.Cu") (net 6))
 (segment (start -3.9 -14.58493) (end 0.5 -10.18493) (width 0.25) (layer "F.Cu") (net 7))
 (segment (start 0.5 -10.18493) (end 0.5 -3.396) (width 0.25) (layer "F.Cu") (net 7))
 (segment (start -3.9 -17.75) (end -3.9 -14.58493) (width 0.25) (layer "F.Cu") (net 7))
 (segment (start 0 -3.396) (end 0 -10.049212) (width 0.25) (layer "F.Cu") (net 2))
 (segment (start 0 -10.049212) (end -5.950788 -16) (width 0.25) (layer "F.Cu") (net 2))
 (segment (start -11.25 -16.75) (end -11.25 -17.75) (width 0.25) (layer "F.Cu") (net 2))
 (segment (start -10.5 -16) (end -11.25 -16.75) (width 0.25) (layer "F.Cu") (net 2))
 (segment (start -5.950788 -16) (end -10.5 -16) (width 0.25) (layer "F.Cu") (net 2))
 (segment (start -12.25 -16.75) (end -11 -15.5) (width 0.25) (layer "F.Cu") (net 3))
 (segment (start -1 -9) (end -1 -3.396) (width 0.25) (layer "F.Cu") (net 3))
 (segment (start -12.25 -17.75) (end -12.25 -16.75) (width 0.25) (layer "F.Cu") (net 3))
 (segment (start -7.5 -15.5) (end -1 -9) (width 0.25) (layer "F.Cu") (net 3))
 (segment (start -11 -15.5) (end -7.5 -15.5) (width 0.25) (layer "F.Cu") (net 3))
 (segment (start 3.501 -14.365282) (end 5.192859 -16.057141) (width 0.25) (layer "F.Cu") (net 15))
 (segment (start 3.501 -3.396) (end 3.501 -11.165762) (width 0.25) (layer "F.Cu") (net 15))
 (segment (start 4 -11.664762) (end 4 -13.866282) (width 0.25) (layer "F.Cu") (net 15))
 (segment (start 11.753213 -16.057141) (end 13 -17.303928) (width 0.25) (layer "F.Cu") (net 15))
 (segment (start 3.501 -11.165762) (end 4 -11.664762) (width 0.25) (layer "F.Cu") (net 15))
 (segment (start 13 -17.303928) (end 13 -17.75) (width 0.25) (layer "F.Cu") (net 15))
 (segment (start 5.192859 -16.057141) (end 11.753213 -16.057141) (width 0.25) (layer "F.Cu") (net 15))
 (segment (start 4 -13.866282) (end 3.501 -14.365282) (width 0.25) (layer "F.Cu") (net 15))
 (segment (start 4.950011 -14.051989) (end 4.950011 -3.845011) (width 0.25) (layer "F.Cu") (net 13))
 (segment (start 12.303693 -15.607621) (end 5.607621 -15.607621) (width 0.25) (layer "F.Cu") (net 13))
 (segment (start 4.950011 -3.845011) (end 4.501 -3.396) (width 0.25) (layer "F.Cu") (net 13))
 (segment (start 14 -17.75) (end 14 -17.303928) (width 0.25) (layer "F.Cu") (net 13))
 (segment (start 14 -17.303928) (end 12.303693 -15.607621) (width 0.25) (layer "F.Cu") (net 13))
 (segment (start 4.501 -14.501) (end 4.950011 -14.051989) (width 0.25) (layer "F.Cu") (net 13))
 (segment (start 5.607621 -15.607621) (end 4.501 -14.501) (width 0.25) (layer "F.Cu") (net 13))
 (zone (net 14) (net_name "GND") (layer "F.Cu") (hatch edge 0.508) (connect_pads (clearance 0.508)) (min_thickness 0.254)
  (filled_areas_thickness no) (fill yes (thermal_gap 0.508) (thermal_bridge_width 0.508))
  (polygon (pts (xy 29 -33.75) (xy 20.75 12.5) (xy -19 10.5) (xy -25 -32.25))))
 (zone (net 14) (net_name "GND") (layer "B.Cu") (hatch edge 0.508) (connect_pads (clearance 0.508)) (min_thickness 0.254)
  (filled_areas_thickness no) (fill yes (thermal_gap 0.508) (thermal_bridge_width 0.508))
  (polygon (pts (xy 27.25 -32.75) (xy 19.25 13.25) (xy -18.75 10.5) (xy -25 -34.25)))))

